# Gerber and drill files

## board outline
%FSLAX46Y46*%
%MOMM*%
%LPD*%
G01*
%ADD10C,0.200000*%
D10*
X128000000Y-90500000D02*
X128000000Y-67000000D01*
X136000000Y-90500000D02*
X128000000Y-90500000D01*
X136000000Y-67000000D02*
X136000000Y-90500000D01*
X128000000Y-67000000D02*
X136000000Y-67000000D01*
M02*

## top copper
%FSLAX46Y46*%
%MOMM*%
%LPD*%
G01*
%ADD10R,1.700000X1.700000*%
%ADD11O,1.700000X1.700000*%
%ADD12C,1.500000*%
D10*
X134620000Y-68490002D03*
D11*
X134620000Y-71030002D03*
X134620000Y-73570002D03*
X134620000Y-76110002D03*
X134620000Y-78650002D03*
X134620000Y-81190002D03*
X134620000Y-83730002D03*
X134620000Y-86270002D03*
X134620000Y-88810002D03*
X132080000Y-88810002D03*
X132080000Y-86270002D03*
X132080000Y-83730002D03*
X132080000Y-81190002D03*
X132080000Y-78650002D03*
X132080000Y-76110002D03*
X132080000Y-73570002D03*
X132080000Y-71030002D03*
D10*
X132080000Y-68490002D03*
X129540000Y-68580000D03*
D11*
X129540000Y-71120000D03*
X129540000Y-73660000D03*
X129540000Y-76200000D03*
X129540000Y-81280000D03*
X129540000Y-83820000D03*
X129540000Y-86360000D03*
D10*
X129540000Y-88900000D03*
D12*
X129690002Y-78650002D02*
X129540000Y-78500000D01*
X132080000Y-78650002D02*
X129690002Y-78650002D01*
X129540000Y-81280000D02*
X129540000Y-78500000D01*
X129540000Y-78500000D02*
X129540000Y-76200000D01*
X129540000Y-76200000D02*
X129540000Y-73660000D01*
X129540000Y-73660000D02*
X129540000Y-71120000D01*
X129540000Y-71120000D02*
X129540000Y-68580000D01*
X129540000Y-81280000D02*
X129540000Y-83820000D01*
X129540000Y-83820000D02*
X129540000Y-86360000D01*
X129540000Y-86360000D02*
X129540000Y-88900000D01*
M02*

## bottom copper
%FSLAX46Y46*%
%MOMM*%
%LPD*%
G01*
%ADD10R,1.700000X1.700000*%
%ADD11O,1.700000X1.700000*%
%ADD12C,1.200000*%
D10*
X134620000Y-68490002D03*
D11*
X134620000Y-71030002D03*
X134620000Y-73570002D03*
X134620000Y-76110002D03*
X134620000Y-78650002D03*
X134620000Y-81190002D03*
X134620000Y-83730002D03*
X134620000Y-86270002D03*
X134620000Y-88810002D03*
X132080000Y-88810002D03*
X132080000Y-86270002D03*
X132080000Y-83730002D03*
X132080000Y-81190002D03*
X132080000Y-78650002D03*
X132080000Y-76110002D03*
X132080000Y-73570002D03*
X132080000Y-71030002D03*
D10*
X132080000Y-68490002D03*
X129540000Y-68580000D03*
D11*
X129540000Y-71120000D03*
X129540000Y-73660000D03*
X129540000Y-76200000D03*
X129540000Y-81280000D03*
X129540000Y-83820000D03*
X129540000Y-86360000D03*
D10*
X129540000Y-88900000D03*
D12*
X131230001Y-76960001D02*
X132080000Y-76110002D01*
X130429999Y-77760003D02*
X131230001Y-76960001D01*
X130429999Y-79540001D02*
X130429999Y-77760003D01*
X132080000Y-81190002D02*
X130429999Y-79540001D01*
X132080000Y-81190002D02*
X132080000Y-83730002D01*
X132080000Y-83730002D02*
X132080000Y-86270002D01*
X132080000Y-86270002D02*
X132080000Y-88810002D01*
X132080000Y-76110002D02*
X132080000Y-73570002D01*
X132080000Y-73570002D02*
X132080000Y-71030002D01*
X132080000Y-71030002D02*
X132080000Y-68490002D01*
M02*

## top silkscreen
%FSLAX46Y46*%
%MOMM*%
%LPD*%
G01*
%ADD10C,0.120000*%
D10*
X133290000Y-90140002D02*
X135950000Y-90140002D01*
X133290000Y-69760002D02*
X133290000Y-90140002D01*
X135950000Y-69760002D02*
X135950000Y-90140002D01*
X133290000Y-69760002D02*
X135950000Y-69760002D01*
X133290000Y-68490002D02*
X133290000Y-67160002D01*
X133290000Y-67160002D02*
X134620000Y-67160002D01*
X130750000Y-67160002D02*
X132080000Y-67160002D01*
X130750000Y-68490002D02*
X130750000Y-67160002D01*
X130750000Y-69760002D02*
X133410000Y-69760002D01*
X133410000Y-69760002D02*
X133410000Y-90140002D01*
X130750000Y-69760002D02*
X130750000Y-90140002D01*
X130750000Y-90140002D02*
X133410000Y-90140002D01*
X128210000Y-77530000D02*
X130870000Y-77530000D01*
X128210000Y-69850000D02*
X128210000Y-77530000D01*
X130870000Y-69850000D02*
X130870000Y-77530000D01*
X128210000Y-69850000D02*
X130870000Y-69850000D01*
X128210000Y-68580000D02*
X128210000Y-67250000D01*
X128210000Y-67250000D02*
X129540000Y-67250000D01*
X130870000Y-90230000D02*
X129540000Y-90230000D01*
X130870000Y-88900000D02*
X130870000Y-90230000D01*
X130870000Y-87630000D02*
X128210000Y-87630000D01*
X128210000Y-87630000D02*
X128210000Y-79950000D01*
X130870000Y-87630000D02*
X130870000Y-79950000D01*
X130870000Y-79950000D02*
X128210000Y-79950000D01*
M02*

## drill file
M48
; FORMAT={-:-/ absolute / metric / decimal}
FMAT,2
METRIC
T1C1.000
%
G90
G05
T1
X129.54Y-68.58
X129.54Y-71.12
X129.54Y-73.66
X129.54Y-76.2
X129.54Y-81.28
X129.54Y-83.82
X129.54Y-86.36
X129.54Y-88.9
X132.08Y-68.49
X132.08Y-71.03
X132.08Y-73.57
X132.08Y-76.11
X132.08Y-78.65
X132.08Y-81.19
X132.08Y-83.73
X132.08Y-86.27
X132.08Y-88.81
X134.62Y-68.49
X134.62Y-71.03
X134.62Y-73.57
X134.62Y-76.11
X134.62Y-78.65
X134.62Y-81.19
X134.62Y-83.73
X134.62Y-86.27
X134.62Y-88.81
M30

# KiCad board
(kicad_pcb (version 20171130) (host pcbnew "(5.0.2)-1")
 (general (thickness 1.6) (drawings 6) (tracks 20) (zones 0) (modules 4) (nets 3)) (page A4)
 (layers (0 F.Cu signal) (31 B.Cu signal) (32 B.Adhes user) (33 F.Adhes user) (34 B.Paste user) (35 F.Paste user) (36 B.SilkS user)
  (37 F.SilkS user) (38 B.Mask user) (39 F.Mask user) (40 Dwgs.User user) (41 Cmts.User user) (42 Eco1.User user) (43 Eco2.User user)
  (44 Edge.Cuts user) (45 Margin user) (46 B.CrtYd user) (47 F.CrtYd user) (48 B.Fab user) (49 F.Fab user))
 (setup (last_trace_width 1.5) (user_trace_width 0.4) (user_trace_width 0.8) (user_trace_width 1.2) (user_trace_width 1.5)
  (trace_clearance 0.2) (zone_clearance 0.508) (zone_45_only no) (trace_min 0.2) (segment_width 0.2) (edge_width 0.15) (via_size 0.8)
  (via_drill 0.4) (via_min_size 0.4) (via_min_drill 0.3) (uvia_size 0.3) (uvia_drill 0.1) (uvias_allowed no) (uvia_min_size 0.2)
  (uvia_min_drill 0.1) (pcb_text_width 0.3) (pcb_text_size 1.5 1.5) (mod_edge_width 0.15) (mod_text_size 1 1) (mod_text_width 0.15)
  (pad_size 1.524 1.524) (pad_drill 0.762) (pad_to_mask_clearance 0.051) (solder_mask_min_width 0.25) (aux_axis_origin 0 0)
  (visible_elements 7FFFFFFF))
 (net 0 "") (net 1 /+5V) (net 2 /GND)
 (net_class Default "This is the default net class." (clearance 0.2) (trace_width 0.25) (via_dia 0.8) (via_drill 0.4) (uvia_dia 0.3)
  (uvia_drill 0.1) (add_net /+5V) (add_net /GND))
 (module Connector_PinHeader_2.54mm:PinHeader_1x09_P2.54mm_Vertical (layer F.Cu) (at 134.62 68.490002)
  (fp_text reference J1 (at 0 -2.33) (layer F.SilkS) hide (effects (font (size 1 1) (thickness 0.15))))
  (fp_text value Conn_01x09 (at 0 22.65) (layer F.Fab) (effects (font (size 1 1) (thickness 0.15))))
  (fp_line (start -1.33 21.65) (end 1.33 21.65) (layer F.SilkS) (width 0.12))
  (fp_line (start -1.33 1.27) (end -1.33 21.65) (layer F.SilkS) (width 0.12))
  (fp_line (start 1.33 1.27) (end 1.33 21.65) (layer F.SilkS) (width 0.12))
  (fp_line (start -1.33 1.27) (end 1.33 1.27) (layer F.SilkS) (width 0.12))
  (fp_line (start -1.33 0) (end -1.33 -1.33) (layer F.SilkS) (width 0.12))
  (fp_line (start -1.33 -1.33) (end 0 -1.33) (layer F.SilkS) (width 0.12))
  (pad 1 thru_hole rect (at 0 0) (size 1.7 1.7) (drill 1) (layers *.Cu *.Mask))
  (pad 2 thru_hole oval (at 0 2.54) (size 1.7 1.7) (drill 1) (layers *.Cu *.Mask))
  (pad 3 thru_hole oval (at 0 5.08) (size 1.7 1.7) (drill 1) (layers *.Cu *.Mask))
  (pad 4 thru_hole oval (at 0 7.62) (size 1.7 1.7) (drill 1) (layers *.Cu *.Mask))
  (pad 5 thru_hole oval (at 0 10.16) (size 1.7 1.7) (drill 1) (layers *.Cu *.Mask))
  (pad 6 thru_hole oval (at 0 12.7) (size 1.7 1.7) (drill 1) (layers *.Cu *.Mask))
  (pad 7 thru_hole oval (at 0 15.24) (size 1.7 1.7) (drill 1) (layers *.Cu *.Mask))
  (pad 8 thru_hole oval (at 0 17.78) (size 1.7 1.7) (drill 1) (layers *.Cu *.Mask))
  (pad 9 thru_hole oval (at 0 20.32) (size 1.7 1.7) (drill 1) (layers *.Cu *.Mask)))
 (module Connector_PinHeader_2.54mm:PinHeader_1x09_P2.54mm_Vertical (layer F.Cu) (at 132.08 68.490002)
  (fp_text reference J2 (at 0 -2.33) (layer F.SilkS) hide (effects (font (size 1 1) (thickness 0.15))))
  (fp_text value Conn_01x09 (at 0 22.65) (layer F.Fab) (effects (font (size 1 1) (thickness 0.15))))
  (fp_line (start -1.33 -1.33) (end 0 -1.33) (layer F.SilkS) (width 0.12))
  (fp_line (start -1.33 0) (end -1.33 -1.33) (layer F.SilkS) (width 0.12))
  (fp_line (start -1.33 1.27) (end 1.33 1.27) (layer F.SilkS) (width 0.12))
  (fp_line (start 1.33 1.27) (end 1.33 21.65) (layer F.SilkS) (width 0.12))
  (fp_line (start -1.33 1.27) (end -1.33 21.65) (layer F.SilkS) (width 0.12))
  (fp_line (start -1.33 21.65) (end 1.33 21.65) (layer F.SilkS) (width 0.12))
  (pad 9 thru_hole oval (at 0 20.32) (size 1.7 1.7) (drill 1) (layers *.Cu *.Mask) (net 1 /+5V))
  (pad 8 thru_hole oval (at 0 17.78) (size 1.7 1.7) (drill 1) (layers *.Cu *.Mask) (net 1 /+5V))
  (pad 7 thru_hole oval (at 0 15.24) (size 1.7 1.7) (drill 1) (layers *.Cu *.Mask) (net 1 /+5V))
  (pad 6 thru_hole oval (at 0 12.7) (size 1.7 1.7) (drill 1) (layers *.Cu *.Mask) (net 1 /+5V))
  (pad 5 thru_hole oval (at 0 10.16) (size 1.7 1.7) (drill 1) (layers *.Cu *.Mask) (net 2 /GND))
  (pad 4 thru_hole oval (at 0 7.62) (size 1.7 1.7) (drill 1) (layers *.Cu *.Mask) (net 1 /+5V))
  (pad 3 thru_hole oval (at 0 5.08) (size 1.7 1.7) (drill 1) (layers *.Cu *.Mask) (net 1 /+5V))
  (pad 2 thru_hole oval (at 0 2.54) (size 1.7 1.7) (drill 1) (layers *.Cu *.Mask) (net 1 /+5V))
  (pad 1 thru_hole rect (at 0 0) (size 1.7 1.7) (drill 1) (layers *.Cu *.Mask) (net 1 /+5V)))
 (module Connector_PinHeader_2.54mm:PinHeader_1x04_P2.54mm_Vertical (layer F.Cu) (at 129.54 68.58)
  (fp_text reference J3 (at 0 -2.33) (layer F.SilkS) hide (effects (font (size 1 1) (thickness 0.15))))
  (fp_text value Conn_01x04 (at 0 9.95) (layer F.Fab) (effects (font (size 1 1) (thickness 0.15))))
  (fp_line (start -1.33 8.95) (end 1.33 8.95) (layer F.SilkS) (width 0.12))
  (fp_line (start -1.33 1.27) (end -1.33 8.95) (layer F.SilkS) (width 0.12))
  (fp_line (start 1.33 1.27) (end 1.33 8.95) (layer F.SilkS) (width 0.12))
  (fp_line (start -1.33 1.27) (end 1.33 1.27) (layer F.SilkS) (width 0.12))
  (fp_line (start -1.33 0) (end -1.33 -1.33) (layer F.SilkS) (width 0.12))
  (fp_line (start -1.33 -1.33) (end 0 -1.33) (layer F.SilkS) (width 0.12))
  (pad 1 thru_hole rect (at 0 0) (size 1.7 1.7) (drill 1) (layers *.Cu *.Mask) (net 2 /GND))
  (pad 2 thru_hole oval (at 0 2.54) (size 1.7 1.7) (drill 1) (layers *.Cu *.Mask) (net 2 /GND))
  (pad 3 thru_hole oval (at 0 5.08) (size 1.7 1.7) (drill 1) (layers *.Cu *.Mask) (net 2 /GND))
  (pad 4 thru_hole oval (at 0 7.62) (size 1.7 1.7) (drill 1) (layers *.Cu *.Mask) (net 2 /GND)))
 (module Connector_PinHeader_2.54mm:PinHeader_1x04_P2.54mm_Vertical (layer F.Cu) (at 129.54 88.9 180)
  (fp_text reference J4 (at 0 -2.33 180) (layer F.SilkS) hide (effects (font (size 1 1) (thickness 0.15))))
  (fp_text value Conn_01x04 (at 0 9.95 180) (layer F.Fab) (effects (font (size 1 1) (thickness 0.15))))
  (fp_line (start -1.33 -1.33) (end 0 -1.33) (layer F.SilkS) (width 0.12))
  (fp_line (start -1.33 0) (end -1.33 -1.33) (layer F.SilkS) (width 0.12))
  (fp_line (start -1.33 1.27) (end 1.33 1.27) (layer F.SilkS) (width 0.12))
  (fp_line (start 1.33 1.27) (end 1.33 8.95) (layer F.SilkS) (width 0.12))
  (fp_line (start -1.33 1.27) (end -1.33 8.95) (layer F.SilkS) (width 0.12))
  (fp_line (start -1.33 8.95) (end 1.33 8.95) (layer F.SilkS) (width 0.12))
  (pad 4 thru_hole oval (at 0 7.62 180) (size 1.7 1.7) (drill 1) (layers *.Cu *.Mask) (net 2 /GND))
  (pad 3 thru_hole oval (at 0 5.08 180) (size 1.7 1.7) (drill 1) (layers *.Cu *.Mask) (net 2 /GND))
  (pad 2 thru_hole oval (at 0 2.54 180) (size 1.7 1.7) (drill 1) (layers *.Cu *.Mask) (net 2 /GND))
  (pad 1 thru_hole rect (at 0 0 180) (size 1.7 1.7) (drill 1) (layers *.Cu *.Mask) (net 2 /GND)))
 (gr_line (start 128 90.5) (end 128 67) (layer Edge.Cuts) (width 0.2))
 (gr_line (start 136 90.5) (end 128 90.5) (layer Edge.Cuts) (width 0.2))
 (gr_line (start 136 67) (end 136 90.5) (layer Edge.Cuts) (width 0.2))
 (gr_line (start 128 67) (end 136 67) (layer Edge.Cuts) (width 0.2))
 (segment (start 131.230001 76.960001) (end 132.08 76.110002) (width 1.2) (layer B.Cu) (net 1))
 (segment (start 130.429999 77.760003) (end 131.230001 76.960001) (width 1.2) (layer B.Cu) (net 1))
 (segment (start 130.429999 79.540001) (end 130.429999 77.760003) (width 1.2) (layer B.Cu) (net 1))
 (segment (start 132.08 81.190002) (end 130.429999 79.540001) (width 1.2) (layer B.Cu) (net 1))
 (segment (start 132.08 81.190002) (end 132.08 83.730002) (width 1.2) (layer B.Cu) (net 1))
 (segment (start 132.08 83.730002) (end 132.08 86.270002) (width 1.2) (layer B.Cu) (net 1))
 (segment (start 132.08 86.270002) (end 132.08 88.810002) (width 1.2) (layer B.Cu) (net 1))
 (segment (start 132.08 76.110002) (end 132.08 73.570002) (width 1.2) (layer B.Cu) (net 1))
 (segment (start 132.08 73.570002) (end 132.08 71.030002) (width 1.2) (layer B.Cu) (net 1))
 (segment (start 132.08 71.030002) (end 132.08 68.490002) (width 1.2) (layer B.Cu) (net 1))
 (segment (start 129.690002 78.650002) (end 129.54 78.5) (width 1.5) (layer F.Cu) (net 2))
 (segment (start 132.08 78.650002) (end 129.690002 78.650002) (width 1.5) (layer F.Cu) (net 2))
 (segment (start 129.54 81.28) (end 129.54 78.5) (width 1.5) (layer F.Cu) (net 2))
 (segment (start 129.54 78.5) (end 129.54 76.2) (width 1.5) (layer F.Cu) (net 2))
 (segment (start 129.54 76.2) (end 129.54 73.66) (width 1.5) (layer F.Cu) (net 2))
 (segment (start 129.54 73.66) (end 129.54 71.12) (width 1.5) (layer F.Cu) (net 2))
 (segment (start 129.54 71.12) (end 129.54 68.58) (width 1.5) (layer F.Cu) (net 2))
 (segment (start 129.54 81.28) (end 129.54 83.82) (width 1.5) (layer F.Cu) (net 2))
 (segment (start 129.54 83.82) (end 129.54 86.36) (width 1.5) (layer F.Cu) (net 2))
 (segment (start 129.54 86.36) (end 129.54 88.9) (width 1.5) (layer F.Cu) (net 2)))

